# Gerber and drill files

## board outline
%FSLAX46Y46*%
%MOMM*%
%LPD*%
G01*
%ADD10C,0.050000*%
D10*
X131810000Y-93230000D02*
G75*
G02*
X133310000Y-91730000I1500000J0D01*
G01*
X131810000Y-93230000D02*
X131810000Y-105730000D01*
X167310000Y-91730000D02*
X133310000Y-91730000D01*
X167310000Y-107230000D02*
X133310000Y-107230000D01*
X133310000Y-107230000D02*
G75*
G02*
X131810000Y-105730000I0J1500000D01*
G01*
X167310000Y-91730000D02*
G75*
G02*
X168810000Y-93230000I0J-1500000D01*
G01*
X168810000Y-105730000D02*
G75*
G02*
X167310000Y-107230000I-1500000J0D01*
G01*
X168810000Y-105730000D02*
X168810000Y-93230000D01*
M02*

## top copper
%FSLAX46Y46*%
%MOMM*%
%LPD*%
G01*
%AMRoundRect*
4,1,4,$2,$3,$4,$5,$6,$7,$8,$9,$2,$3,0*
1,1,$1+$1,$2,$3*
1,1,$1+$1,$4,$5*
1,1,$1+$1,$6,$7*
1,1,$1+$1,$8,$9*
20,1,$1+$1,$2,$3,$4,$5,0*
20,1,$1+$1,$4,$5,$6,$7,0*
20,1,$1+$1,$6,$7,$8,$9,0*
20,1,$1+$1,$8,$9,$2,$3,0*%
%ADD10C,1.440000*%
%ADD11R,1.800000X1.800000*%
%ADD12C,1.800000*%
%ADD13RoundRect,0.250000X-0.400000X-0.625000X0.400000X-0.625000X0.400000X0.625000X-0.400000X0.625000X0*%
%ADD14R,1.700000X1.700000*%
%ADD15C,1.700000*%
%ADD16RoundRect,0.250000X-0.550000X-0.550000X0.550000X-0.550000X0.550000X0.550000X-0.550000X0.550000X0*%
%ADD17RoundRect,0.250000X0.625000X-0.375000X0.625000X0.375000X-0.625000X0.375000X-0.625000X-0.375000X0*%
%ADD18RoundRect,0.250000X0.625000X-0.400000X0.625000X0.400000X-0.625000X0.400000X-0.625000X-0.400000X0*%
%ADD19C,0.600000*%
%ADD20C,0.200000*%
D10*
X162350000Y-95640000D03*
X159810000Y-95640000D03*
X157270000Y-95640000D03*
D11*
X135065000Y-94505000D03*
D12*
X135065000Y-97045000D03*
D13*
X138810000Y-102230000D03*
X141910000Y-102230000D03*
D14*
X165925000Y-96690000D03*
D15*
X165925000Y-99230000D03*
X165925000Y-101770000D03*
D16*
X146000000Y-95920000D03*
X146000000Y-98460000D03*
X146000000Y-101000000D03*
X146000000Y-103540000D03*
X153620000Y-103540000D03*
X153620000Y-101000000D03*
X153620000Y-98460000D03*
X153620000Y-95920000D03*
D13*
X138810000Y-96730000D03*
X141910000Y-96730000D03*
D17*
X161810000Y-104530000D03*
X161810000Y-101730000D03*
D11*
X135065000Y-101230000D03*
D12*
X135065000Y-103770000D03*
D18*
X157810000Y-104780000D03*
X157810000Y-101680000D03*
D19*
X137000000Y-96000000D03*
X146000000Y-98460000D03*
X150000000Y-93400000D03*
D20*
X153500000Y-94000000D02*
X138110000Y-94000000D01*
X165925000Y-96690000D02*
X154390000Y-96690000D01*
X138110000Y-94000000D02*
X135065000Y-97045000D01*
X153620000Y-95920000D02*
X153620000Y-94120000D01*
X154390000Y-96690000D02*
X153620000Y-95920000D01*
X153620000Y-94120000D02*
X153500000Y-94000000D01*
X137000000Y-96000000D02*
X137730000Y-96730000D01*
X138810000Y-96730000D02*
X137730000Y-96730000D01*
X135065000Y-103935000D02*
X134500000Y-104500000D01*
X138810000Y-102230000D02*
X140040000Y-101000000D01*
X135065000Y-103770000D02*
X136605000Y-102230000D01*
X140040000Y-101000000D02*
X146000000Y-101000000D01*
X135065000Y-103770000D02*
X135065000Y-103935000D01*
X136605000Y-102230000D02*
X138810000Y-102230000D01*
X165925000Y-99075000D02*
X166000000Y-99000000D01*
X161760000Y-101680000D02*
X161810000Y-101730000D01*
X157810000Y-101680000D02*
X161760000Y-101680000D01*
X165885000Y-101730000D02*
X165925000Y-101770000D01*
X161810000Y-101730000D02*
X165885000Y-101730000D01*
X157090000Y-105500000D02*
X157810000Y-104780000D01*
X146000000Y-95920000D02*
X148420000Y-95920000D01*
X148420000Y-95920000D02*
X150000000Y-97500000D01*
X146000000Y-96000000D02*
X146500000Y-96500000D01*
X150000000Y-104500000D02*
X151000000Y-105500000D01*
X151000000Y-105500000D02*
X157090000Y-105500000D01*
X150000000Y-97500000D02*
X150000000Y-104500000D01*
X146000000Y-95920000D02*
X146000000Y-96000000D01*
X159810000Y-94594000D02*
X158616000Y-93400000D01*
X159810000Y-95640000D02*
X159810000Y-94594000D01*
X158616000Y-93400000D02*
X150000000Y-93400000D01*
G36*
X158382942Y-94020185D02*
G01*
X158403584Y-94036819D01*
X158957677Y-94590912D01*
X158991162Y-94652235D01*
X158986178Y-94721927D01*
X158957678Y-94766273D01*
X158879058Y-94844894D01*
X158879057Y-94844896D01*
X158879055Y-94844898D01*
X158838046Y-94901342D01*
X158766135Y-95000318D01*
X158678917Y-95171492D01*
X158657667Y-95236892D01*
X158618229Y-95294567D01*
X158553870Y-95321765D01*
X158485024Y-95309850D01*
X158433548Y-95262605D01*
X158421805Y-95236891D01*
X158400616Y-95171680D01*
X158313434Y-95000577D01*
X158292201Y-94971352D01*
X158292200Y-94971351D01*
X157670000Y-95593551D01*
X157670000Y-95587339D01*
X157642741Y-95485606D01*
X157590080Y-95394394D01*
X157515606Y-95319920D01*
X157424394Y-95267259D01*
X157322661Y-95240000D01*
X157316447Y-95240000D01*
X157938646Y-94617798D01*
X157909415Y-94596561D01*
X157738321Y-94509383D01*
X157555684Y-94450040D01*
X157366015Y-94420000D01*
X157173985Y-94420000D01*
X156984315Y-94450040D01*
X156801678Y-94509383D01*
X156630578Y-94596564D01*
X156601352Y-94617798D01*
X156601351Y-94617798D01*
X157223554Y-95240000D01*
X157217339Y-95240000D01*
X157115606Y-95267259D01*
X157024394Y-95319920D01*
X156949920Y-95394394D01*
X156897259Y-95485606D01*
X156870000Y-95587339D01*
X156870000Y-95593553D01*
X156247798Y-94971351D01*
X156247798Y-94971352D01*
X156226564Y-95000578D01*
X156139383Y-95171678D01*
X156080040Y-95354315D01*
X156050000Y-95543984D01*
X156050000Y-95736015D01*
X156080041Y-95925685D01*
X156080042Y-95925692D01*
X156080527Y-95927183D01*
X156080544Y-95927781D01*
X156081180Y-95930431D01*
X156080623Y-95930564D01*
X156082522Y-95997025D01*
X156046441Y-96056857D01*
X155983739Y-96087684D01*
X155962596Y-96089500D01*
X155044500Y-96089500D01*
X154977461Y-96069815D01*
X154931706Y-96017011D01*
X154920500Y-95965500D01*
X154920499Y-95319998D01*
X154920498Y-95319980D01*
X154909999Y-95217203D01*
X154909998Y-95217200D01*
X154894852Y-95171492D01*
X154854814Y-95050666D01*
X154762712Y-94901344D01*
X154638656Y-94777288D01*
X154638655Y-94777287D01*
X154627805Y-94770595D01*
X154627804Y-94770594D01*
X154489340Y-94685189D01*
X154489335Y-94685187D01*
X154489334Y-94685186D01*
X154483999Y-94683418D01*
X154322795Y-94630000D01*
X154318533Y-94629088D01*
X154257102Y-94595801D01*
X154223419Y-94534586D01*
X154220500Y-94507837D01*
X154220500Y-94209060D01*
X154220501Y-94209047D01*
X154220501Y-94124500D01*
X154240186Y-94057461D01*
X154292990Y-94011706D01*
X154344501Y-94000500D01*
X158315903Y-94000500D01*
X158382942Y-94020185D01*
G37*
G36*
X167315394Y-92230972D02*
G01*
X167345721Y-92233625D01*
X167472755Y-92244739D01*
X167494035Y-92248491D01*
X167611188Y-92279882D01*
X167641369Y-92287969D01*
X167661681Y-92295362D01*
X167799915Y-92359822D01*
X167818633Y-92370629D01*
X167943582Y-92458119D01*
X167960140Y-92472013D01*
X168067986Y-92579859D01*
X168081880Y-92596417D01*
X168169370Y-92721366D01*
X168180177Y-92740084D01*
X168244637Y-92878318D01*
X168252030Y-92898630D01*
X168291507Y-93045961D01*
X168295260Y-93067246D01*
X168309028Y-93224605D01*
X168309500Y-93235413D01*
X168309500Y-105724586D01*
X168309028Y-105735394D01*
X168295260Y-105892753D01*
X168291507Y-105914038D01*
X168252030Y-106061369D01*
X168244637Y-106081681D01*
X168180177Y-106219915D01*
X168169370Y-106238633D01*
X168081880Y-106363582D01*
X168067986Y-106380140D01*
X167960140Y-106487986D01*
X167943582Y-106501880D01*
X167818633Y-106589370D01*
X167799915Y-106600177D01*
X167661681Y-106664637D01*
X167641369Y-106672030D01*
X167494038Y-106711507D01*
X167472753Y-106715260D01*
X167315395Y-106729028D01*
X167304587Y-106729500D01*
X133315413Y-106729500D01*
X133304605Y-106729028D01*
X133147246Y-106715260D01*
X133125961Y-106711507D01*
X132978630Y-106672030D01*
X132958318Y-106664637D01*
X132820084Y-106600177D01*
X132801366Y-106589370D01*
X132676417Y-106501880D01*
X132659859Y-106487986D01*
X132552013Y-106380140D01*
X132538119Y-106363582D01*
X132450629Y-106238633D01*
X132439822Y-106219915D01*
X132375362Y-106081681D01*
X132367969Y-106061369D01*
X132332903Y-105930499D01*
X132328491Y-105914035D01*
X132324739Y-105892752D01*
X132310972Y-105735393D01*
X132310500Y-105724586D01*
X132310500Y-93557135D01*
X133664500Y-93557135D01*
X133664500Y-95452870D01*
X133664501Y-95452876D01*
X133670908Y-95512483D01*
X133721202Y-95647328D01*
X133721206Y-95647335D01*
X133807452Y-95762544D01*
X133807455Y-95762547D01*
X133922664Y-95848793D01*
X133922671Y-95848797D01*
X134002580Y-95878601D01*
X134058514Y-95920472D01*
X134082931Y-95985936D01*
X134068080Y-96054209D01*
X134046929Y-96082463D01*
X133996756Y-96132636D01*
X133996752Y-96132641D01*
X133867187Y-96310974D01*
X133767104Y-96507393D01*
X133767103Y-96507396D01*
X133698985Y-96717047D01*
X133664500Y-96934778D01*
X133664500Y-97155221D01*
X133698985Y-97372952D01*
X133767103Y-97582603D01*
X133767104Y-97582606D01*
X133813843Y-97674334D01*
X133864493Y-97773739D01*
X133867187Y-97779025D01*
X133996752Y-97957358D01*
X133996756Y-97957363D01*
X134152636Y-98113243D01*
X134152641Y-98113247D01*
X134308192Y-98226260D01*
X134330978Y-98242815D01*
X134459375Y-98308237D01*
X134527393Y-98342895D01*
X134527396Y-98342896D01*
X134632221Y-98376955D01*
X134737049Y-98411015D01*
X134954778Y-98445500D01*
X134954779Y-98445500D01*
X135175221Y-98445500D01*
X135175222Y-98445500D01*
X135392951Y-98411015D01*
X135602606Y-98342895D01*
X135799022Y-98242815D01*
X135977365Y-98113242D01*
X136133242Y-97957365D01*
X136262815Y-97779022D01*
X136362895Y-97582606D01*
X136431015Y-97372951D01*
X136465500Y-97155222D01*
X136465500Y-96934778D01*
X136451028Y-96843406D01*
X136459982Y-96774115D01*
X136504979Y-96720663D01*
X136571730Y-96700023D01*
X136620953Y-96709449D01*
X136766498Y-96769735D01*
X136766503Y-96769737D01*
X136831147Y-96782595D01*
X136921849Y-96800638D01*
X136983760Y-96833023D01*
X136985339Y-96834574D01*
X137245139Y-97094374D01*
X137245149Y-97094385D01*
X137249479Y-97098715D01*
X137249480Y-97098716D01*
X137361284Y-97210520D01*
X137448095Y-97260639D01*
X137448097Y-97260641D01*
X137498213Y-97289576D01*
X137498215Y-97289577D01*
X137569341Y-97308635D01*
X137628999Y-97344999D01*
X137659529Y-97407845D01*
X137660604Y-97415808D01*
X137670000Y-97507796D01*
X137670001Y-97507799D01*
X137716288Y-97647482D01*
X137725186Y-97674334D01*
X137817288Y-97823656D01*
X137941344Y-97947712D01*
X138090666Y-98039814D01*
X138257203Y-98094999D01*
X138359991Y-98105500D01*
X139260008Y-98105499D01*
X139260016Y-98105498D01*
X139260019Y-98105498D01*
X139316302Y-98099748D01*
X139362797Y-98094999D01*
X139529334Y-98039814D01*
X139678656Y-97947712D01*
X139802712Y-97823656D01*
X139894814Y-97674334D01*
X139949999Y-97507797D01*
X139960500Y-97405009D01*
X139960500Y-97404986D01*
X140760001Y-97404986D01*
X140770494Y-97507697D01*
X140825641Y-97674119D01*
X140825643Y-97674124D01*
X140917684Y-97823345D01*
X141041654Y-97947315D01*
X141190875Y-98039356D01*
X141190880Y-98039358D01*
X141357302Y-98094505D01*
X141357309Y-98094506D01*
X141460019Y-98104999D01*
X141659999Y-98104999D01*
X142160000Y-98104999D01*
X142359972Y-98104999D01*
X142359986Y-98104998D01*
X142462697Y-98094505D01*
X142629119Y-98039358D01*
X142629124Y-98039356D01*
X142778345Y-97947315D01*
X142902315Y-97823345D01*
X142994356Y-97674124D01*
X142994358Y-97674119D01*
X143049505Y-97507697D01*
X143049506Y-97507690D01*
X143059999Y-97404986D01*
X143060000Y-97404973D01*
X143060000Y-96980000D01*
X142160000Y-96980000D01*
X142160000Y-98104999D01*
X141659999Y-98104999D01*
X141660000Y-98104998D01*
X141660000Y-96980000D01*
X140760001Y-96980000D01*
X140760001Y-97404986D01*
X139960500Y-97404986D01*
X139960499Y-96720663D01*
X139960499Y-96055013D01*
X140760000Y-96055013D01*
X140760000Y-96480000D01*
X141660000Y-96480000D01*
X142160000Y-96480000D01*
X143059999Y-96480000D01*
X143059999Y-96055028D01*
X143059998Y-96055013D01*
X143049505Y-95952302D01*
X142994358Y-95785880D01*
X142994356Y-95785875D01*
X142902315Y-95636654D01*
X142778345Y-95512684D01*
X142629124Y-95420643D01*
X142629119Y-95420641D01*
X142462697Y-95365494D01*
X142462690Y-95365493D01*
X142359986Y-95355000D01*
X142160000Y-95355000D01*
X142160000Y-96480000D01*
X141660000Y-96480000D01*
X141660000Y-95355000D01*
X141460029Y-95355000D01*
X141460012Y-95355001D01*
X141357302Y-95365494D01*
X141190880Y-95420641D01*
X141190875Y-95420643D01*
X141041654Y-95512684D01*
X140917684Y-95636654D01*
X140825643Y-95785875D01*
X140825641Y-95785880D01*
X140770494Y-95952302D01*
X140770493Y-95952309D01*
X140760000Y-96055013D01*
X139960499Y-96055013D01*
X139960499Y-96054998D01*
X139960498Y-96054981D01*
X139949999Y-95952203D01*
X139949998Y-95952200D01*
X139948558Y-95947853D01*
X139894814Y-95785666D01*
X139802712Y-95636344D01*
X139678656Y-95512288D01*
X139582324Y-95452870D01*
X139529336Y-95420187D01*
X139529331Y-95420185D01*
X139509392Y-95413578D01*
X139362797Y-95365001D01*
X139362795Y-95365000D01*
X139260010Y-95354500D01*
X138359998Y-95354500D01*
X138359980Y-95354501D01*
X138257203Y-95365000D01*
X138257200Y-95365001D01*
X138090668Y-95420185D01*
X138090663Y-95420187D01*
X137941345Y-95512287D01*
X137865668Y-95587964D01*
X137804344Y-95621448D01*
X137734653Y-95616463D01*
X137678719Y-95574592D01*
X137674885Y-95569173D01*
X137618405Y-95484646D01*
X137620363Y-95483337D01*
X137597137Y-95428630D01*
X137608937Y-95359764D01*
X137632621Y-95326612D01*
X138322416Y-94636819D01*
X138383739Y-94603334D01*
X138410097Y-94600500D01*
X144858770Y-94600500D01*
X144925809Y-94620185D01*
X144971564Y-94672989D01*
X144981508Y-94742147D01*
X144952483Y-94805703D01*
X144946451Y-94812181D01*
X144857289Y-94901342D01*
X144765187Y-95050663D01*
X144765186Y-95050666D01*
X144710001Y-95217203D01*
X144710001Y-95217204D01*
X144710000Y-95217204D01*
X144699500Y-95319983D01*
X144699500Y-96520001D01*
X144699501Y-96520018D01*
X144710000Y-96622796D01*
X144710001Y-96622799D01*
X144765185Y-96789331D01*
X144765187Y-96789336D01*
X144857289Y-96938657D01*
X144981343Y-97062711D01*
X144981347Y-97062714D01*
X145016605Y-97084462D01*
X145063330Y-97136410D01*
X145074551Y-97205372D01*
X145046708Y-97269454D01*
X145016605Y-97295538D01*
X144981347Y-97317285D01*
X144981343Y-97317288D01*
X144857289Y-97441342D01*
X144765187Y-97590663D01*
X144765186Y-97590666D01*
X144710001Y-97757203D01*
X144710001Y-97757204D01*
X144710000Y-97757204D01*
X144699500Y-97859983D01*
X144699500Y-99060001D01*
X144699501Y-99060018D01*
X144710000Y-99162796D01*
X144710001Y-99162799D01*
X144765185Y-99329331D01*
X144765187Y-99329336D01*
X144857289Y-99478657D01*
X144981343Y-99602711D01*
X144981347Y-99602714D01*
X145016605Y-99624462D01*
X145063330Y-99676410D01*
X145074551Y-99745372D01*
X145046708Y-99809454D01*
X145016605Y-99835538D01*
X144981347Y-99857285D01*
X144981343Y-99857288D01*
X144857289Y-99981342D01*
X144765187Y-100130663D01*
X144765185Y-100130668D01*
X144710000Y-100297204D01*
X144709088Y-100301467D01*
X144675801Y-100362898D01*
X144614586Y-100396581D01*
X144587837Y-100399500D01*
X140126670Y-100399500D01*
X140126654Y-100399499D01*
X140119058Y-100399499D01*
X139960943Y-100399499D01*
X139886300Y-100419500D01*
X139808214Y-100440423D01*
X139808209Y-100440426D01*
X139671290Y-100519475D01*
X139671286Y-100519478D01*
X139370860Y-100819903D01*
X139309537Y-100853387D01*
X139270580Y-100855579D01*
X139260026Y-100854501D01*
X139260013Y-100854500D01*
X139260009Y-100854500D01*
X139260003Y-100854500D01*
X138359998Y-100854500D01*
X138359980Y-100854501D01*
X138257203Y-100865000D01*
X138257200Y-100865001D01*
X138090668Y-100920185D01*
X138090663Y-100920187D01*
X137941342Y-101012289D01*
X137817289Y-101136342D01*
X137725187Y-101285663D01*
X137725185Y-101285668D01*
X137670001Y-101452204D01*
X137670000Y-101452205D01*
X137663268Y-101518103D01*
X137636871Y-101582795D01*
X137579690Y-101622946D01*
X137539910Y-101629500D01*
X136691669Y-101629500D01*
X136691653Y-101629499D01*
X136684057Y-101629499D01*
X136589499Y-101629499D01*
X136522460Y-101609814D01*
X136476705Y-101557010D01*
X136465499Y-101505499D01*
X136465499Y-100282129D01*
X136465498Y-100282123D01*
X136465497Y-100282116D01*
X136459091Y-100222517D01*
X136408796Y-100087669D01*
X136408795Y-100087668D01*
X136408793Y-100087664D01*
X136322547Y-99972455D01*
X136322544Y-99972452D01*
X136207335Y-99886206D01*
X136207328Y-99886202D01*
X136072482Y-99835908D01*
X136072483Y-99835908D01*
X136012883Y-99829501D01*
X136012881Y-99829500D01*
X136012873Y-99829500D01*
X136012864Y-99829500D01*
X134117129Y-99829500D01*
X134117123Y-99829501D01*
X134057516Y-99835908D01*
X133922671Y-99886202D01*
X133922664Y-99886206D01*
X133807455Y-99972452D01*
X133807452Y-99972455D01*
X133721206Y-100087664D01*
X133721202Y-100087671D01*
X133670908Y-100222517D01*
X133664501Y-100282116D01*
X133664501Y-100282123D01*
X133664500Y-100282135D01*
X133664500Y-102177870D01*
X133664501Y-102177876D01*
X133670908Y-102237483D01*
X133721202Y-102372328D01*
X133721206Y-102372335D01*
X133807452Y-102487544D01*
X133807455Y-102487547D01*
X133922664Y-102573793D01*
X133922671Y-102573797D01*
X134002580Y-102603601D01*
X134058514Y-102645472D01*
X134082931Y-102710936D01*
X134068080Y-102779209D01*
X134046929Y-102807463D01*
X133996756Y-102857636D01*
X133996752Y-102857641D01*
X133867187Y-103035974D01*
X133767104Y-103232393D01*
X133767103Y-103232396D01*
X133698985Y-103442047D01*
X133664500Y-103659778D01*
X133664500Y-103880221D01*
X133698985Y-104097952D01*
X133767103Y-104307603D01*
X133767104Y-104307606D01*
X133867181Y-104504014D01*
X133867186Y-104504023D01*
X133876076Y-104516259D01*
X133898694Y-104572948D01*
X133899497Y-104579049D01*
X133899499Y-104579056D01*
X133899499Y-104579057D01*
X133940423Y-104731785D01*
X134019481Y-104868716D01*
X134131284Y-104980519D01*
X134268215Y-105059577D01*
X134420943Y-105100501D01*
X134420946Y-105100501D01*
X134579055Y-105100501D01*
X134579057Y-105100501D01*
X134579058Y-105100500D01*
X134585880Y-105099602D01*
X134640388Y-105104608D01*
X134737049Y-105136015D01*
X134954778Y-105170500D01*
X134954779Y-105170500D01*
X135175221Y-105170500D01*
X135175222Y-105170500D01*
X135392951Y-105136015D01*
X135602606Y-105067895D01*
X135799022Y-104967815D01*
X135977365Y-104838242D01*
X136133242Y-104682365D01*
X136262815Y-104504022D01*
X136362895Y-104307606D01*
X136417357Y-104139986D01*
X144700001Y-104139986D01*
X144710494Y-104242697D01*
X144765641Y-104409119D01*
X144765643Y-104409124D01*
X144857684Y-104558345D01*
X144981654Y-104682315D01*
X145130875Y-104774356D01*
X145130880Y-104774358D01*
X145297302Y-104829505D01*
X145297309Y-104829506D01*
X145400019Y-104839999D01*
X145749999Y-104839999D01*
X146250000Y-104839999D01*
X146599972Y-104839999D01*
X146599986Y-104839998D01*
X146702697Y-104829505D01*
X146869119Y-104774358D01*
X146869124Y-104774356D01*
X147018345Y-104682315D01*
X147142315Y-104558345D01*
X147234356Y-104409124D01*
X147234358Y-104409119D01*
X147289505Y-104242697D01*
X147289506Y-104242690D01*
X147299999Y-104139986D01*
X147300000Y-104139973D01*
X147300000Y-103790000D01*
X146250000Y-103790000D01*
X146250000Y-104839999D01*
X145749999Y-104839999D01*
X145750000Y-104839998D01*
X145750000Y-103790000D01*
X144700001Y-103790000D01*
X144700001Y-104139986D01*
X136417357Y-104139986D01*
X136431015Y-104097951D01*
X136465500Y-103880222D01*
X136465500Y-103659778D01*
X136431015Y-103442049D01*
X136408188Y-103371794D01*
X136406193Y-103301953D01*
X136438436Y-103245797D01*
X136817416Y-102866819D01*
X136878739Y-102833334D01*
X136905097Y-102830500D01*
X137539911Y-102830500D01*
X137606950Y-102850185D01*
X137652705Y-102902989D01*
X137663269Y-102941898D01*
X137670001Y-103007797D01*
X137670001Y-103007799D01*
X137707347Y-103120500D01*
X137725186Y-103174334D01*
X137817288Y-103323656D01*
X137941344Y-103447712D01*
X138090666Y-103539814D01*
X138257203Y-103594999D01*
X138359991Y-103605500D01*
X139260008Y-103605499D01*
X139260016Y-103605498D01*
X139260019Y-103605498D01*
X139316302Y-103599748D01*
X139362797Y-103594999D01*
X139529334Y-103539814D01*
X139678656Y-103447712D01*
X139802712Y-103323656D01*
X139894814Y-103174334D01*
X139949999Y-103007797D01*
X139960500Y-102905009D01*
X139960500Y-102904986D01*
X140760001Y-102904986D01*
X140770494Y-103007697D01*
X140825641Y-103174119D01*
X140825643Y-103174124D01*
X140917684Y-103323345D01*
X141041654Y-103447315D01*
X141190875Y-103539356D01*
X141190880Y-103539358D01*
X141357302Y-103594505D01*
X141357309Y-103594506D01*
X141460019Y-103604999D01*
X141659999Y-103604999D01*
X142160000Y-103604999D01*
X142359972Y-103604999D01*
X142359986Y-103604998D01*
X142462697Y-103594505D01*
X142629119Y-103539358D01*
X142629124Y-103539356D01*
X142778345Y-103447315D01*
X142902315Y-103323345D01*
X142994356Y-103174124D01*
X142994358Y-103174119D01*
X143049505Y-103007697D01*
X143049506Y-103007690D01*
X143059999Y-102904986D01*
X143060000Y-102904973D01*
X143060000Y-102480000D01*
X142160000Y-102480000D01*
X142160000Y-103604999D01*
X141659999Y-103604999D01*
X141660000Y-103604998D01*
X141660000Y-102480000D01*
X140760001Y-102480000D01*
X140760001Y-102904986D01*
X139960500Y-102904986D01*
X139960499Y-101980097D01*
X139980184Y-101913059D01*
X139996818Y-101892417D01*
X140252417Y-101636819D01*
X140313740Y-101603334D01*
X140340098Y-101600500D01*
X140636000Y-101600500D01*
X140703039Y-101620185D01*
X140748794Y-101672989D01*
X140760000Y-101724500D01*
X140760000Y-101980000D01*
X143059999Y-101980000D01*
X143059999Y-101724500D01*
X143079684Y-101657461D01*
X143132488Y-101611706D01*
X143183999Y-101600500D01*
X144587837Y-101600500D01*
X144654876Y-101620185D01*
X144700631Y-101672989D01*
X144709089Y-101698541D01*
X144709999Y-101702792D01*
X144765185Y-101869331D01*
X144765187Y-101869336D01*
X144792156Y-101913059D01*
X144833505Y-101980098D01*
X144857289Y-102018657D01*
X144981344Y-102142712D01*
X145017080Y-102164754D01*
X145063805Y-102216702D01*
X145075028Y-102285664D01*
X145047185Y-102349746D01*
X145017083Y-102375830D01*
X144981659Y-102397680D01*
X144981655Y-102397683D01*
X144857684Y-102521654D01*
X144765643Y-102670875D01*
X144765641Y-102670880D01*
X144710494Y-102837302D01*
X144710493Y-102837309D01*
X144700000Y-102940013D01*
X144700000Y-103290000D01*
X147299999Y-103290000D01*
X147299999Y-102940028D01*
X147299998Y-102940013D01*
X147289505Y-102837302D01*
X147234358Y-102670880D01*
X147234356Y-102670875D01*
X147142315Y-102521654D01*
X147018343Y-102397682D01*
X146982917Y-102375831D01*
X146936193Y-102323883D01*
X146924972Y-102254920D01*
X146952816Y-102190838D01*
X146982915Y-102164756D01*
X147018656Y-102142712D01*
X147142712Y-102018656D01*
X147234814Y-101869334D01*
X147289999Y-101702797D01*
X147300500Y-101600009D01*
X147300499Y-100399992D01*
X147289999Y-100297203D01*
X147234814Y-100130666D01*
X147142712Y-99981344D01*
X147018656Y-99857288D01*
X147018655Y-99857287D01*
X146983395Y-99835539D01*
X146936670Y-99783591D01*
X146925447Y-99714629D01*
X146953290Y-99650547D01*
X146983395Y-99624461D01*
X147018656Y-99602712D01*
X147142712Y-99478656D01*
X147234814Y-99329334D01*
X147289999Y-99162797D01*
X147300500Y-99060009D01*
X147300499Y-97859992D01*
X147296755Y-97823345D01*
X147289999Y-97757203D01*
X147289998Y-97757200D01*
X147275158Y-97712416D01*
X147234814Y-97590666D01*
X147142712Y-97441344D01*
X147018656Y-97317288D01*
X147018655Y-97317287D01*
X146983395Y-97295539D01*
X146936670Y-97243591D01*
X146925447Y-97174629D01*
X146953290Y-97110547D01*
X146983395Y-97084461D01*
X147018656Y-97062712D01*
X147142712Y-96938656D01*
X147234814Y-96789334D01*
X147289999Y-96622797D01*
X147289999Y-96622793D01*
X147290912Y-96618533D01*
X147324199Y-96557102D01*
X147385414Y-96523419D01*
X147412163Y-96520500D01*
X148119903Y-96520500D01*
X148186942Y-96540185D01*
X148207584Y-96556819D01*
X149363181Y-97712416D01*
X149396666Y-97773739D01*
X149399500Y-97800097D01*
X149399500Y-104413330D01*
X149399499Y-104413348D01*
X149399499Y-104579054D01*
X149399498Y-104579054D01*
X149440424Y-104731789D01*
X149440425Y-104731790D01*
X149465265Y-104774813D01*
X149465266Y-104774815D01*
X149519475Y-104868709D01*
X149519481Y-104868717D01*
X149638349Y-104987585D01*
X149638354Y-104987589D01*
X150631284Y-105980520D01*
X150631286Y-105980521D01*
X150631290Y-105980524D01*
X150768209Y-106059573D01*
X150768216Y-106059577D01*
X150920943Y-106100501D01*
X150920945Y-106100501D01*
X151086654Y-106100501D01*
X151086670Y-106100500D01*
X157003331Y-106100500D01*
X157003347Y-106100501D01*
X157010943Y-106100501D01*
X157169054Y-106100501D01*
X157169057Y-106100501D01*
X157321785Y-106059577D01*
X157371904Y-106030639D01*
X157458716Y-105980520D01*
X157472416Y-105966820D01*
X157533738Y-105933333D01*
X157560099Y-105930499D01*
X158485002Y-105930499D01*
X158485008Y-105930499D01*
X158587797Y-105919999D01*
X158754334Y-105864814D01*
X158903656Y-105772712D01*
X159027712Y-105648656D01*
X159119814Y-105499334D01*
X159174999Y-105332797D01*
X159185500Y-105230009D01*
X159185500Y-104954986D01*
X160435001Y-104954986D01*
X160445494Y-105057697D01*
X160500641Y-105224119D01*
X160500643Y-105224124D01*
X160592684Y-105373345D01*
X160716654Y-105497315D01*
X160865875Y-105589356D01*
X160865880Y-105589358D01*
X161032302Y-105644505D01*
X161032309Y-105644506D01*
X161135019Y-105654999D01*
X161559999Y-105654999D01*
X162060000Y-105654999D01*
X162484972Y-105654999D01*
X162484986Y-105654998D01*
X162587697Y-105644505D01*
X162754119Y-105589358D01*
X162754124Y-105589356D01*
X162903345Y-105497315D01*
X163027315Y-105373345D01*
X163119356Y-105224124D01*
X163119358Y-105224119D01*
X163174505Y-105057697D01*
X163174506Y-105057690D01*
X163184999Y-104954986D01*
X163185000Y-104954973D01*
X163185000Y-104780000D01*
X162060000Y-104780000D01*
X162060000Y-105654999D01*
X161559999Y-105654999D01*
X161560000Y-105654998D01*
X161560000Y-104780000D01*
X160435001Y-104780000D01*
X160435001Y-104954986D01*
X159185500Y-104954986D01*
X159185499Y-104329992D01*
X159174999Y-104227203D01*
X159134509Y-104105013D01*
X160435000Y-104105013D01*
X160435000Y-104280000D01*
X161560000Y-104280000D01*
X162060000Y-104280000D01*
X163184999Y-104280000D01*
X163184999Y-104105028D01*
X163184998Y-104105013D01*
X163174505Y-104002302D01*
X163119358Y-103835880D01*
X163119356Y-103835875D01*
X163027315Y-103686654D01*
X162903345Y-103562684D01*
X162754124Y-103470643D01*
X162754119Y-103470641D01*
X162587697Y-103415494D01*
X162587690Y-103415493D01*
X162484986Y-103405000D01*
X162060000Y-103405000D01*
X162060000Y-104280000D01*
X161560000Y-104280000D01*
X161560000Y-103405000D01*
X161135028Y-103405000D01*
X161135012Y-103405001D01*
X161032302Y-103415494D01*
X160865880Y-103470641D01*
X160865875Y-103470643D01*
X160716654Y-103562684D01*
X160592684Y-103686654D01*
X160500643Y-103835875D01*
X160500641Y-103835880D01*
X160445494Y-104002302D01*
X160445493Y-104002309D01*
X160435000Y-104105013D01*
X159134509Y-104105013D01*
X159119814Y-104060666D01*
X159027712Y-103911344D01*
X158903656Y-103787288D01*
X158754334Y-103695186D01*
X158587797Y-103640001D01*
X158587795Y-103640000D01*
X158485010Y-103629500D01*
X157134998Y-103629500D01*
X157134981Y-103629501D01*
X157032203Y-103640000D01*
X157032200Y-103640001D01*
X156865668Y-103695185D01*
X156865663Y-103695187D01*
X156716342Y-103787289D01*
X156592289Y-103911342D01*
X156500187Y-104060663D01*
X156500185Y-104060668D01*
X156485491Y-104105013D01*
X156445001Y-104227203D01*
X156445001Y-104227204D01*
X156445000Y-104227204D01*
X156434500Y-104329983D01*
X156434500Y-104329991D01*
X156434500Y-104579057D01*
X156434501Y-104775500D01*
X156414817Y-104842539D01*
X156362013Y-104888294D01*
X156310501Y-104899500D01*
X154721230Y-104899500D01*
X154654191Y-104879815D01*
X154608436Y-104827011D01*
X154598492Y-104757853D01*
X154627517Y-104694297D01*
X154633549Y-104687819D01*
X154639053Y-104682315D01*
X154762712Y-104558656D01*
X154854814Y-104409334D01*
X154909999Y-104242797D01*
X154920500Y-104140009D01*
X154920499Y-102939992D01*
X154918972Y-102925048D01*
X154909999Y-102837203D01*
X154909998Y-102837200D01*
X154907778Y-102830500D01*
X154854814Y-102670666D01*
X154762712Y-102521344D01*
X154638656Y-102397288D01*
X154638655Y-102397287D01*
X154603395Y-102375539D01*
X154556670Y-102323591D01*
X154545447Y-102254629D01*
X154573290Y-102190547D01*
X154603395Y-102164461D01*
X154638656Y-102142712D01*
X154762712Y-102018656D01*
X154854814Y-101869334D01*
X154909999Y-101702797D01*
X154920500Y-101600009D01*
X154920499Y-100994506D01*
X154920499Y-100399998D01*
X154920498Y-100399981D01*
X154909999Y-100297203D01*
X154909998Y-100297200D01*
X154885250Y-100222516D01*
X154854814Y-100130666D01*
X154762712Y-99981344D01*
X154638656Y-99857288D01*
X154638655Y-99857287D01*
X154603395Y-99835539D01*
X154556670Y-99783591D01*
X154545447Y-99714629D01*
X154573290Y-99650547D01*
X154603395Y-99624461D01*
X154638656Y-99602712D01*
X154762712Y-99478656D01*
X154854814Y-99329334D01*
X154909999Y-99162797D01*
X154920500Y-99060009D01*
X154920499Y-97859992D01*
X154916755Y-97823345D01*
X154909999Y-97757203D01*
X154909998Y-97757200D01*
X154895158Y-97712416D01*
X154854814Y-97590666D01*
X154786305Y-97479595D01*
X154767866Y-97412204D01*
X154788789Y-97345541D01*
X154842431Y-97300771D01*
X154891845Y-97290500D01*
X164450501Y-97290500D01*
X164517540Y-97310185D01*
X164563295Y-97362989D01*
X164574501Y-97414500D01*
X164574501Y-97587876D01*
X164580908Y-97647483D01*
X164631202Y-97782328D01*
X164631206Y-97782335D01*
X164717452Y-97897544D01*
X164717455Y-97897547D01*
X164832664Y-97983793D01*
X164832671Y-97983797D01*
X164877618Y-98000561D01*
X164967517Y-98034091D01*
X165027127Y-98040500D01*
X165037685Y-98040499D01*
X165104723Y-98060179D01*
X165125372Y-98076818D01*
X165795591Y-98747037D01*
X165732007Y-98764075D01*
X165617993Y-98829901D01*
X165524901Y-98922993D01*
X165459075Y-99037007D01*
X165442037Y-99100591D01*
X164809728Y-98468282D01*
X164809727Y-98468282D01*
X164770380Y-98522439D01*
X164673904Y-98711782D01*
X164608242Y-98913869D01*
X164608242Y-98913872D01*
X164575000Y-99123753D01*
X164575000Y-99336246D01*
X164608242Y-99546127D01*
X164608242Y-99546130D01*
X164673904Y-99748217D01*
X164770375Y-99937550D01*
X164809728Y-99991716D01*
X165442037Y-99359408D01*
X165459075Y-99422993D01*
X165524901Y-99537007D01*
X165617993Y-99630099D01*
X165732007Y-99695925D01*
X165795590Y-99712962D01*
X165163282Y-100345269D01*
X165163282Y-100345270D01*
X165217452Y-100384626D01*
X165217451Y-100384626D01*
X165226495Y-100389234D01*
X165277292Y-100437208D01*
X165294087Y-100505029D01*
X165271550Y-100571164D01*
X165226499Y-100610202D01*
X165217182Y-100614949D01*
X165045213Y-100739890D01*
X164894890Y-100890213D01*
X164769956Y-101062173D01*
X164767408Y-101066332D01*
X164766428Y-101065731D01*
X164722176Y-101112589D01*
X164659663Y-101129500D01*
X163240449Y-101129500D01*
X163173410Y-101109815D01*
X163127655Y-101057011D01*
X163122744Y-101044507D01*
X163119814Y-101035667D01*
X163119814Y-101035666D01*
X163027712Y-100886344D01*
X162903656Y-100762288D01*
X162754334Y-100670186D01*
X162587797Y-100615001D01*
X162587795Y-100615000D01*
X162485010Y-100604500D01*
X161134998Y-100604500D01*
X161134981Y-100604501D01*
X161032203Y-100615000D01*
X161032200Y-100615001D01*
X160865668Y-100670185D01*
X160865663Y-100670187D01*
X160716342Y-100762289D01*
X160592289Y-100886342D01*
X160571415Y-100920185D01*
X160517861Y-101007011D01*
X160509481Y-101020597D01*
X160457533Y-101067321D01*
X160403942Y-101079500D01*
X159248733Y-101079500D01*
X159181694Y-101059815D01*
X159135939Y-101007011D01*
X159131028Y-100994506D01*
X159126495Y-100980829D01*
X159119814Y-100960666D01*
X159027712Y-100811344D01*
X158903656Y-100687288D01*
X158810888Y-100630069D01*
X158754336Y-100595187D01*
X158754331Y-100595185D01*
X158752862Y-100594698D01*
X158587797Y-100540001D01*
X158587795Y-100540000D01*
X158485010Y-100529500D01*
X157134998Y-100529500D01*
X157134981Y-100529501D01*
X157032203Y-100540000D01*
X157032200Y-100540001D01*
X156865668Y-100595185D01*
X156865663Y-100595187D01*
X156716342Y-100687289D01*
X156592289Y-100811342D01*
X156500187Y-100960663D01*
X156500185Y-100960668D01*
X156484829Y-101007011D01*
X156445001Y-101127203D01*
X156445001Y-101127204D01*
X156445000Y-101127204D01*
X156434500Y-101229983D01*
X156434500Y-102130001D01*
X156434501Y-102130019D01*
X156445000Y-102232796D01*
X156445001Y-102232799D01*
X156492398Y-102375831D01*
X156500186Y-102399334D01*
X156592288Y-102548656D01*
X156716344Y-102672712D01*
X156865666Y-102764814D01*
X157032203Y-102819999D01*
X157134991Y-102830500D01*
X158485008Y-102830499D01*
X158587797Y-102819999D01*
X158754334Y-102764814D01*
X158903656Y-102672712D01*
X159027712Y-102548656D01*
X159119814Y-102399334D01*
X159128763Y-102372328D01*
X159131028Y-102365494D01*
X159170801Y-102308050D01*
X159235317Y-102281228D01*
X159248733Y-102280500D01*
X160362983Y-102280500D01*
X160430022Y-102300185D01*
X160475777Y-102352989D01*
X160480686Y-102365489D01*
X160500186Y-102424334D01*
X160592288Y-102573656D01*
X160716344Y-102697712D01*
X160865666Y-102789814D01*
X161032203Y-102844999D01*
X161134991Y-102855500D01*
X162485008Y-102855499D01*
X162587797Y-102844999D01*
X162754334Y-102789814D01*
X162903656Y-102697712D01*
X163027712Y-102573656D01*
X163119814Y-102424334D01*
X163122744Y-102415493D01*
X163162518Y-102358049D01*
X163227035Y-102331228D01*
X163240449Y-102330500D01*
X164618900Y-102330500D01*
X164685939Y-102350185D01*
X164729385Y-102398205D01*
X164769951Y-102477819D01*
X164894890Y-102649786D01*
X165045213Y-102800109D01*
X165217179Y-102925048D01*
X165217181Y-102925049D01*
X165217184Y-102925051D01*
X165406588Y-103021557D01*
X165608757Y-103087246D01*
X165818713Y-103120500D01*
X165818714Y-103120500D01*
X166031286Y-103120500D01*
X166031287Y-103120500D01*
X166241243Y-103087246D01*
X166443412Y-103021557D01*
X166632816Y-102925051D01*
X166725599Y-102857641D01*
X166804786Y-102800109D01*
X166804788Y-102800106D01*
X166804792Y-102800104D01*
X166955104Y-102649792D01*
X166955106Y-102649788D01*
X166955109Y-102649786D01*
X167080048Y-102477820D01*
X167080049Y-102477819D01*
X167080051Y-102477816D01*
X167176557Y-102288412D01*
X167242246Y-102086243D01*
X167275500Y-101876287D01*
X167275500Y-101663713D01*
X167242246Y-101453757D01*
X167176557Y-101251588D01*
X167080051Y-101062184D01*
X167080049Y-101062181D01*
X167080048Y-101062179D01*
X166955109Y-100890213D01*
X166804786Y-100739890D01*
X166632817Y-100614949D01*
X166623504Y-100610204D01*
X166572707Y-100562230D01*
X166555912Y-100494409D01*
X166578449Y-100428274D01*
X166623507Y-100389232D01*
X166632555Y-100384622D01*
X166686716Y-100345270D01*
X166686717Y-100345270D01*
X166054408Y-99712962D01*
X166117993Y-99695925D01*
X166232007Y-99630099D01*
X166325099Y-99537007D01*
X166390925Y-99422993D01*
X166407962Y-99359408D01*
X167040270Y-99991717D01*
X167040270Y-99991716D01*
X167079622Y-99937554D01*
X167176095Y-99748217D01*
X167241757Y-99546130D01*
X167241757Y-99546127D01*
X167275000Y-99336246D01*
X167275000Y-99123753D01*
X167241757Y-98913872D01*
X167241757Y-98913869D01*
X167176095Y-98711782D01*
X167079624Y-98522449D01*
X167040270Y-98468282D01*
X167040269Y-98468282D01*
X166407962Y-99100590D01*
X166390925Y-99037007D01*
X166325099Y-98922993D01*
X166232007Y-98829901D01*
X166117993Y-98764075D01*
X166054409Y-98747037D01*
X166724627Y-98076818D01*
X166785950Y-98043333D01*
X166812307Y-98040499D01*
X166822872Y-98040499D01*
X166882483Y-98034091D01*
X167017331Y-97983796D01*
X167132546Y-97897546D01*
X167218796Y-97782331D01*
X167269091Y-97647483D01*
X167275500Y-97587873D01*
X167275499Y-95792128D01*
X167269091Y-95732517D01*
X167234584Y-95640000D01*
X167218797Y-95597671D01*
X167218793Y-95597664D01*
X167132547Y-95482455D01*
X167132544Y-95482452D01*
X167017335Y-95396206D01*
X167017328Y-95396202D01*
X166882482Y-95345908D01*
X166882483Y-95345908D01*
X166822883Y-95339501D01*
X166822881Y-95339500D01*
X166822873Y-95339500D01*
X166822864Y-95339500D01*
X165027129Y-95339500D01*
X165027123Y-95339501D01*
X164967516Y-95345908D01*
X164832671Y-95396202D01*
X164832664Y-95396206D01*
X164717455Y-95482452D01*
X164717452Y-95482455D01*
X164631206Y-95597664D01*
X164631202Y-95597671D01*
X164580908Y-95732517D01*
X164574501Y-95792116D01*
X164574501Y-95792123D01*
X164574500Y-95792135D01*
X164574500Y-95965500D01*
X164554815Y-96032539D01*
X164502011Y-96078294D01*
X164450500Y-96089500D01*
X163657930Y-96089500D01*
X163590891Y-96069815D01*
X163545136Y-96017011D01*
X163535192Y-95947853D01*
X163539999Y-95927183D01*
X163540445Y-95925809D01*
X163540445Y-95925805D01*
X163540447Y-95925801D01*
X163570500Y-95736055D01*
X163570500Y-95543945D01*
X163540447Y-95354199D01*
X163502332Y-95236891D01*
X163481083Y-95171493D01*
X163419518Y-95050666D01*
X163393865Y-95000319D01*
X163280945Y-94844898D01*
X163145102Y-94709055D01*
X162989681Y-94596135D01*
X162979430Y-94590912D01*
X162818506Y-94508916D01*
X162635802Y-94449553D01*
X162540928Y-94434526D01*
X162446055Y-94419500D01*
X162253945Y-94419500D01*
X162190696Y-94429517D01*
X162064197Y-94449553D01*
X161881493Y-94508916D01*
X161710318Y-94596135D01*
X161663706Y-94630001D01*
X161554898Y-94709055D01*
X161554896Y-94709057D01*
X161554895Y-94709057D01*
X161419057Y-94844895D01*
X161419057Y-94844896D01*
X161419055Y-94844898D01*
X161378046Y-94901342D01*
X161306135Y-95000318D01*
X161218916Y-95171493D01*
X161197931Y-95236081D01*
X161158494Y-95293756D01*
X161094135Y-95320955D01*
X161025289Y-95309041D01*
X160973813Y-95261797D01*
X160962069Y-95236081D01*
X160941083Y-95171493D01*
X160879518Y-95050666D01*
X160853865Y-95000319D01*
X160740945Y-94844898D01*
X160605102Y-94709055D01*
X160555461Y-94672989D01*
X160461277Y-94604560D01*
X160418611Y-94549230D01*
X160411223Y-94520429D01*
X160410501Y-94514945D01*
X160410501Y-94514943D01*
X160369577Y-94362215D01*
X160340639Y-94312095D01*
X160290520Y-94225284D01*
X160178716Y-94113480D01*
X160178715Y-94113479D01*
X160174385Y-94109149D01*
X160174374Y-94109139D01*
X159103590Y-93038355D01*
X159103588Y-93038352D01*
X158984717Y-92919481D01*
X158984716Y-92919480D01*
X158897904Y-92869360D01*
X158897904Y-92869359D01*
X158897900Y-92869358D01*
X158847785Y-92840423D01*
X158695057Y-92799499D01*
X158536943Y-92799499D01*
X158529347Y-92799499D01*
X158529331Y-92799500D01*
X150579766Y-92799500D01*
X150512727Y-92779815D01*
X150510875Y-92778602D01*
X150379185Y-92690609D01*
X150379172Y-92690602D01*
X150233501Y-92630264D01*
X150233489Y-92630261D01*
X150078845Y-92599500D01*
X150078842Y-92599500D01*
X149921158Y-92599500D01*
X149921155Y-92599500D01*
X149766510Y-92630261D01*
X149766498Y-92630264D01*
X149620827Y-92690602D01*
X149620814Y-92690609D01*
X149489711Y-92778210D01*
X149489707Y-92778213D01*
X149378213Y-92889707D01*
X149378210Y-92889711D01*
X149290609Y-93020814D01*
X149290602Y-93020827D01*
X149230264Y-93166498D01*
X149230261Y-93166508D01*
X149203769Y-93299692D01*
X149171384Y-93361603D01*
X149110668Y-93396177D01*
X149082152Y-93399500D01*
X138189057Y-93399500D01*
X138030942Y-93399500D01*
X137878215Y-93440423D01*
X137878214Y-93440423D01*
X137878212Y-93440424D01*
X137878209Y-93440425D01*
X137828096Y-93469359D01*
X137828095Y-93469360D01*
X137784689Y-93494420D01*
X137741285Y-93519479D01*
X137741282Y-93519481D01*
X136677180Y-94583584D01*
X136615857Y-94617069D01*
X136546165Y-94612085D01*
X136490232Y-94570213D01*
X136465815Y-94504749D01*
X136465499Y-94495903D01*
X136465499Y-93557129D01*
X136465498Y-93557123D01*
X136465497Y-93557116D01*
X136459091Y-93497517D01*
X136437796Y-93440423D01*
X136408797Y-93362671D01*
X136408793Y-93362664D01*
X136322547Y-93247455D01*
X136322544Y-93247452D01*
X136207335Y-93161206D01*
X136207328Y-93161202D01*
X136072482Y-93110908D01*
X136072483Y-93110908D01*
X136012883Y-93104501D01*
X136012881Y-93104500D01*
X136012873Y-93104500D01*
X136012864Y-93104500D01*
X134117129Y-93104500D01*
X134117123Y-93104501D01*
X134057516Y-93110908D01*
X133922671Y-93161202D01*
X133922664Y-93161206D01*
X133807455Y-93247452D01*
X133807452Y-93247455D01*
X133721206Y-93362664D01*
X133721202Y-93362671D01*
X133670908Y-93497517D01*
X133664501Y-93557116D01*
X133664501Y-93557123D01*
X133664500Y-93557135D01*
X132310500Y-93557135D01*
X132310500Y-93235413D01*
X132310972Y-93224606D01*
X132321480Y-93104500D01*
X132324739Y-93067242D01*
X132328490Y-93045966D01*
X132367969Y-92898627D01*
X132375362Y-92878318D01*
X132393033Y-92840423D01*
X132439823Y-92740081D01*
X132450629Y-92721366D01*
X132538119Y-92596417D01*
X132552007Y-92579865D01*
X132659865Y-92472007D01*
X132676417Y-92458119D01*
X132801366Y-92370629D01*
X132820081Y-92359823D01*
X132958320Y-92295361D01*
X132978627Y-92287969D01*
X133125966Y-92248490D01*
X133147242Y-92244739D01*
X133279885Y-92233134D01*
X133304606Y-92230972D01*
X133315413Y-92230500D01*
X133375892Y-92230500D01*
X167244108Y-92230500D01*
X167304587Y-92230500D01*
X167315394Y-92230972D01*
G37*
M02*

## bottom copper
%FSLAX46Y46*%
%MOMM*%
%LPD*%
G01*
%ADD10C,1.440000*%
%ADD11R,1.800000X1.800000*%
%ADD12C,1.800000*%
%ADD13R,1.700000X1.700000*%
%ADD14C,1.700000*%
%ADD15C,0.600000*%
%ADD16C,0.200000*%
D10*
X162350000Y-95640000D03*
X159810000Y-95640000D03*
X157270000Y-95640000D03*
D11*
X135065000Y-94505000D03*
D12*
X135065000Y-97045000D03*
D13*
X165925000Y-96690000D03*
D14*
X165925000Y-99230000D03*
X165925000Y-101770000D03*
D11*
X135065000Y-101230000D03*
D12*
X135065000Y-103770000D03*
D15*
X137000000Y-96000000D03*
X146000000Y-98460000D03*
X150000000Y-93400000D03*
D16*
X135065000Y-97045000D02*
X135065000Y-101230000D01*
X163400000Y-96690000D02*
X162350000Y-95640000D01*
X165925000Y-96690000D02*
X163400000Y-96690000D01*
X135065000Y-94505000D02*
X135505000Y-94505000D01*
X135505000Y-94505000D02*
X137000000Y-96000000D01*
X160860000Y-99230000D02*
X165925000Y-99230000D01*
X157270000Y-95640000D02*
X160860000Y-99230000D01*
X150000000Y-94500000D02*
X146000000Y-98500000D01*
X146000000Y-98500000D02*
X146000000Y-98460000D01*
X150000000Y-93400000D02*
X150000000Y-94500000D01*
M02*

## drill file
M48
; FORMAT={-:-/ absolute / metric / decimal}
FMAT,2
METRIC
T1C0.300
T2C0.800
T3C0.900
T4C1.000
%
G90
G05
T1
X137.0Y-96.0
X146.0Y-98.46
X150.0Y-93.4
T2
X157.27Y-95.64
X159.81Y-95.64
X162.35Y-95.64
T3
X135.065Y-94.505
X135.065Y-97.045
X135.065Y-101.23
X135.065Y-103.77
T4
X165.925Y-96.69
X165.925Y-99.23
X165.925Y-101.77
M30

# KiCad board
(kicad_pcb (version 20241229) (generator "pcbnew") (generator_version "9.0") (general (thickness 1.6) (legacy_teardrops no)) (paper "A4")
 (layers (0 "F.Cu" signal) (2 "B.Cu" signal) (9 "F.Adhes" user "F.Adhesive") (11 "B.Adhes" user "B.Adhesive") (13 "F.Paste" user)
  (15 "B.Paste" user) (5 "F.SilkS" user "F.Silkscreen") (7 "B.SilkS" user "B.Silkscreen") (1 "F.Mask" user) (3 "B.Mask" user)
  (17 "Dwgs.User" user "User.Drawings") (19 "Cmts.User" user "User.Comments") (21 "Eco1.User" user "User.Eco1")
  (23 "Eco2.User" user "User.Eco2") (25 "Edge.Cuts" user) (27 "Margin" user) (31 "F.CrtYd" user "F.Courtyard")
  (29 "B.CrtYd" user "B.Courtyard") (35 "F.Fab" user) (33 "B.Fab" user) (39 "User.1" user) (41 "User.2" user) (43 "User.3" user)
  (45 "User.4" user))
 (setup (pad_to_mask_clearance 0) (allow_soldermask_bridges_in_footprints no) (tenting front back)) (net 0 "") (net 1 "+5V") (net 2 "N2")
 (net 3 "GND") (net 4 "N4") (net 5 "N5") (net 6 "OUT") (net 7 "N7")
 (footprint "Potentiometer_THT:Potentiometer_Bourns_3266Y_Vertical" (layer "F.Cu") (at 162.35 95.64)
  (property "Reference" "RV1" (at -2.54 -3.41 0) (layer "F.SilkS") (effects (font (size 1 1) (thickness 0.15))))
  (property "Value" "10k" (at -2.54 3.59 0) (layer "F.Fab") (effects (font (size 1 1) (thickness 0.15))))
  (pad "1" thru_hole circle (at 0 0) (size 1.44 1.44) (drill 0.8) (layers "*.Cu" "*.Mask") (remove_unused_layers no) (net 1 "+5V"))
  (pad "2" thru_hole circle (at -2.54 0) (size 1.44 1.44) (drill 0.8) (layers "*.Cu" "*.Mask") (remove_unused_layers no) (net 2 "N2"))
  (pad "3" thru_hole circle (at -5.08 0) (size 1.44 1.44) (drill 0.8) (layers "*.Cu" "*.Mask") (remove_unused_layers no) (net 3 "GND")))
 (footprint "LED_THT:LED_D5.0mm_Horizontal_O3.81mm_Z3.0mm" (layer "F.Cu") (at 135.065 94.505 -90)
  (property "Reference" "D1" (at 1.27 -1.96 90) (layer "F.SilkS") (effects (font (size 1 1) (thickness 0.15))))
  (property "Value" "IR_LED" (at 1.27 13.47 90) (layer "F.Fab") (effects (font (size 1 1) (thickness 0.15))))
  (pad "1" thru_hole rect (at 0 0 270) (size 1.8 1.8) (drill 0.9) (layers "*.Cu" "*.Mask") (remove_unused_layers no) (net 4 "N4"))
  (pad "2" thru_hole circle (at 2.54 0 270) (size 1.8 1.8) (drill 0.9) (layers "*.Cu" "*.Mask") (remove_unused_layers no) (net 1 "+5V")))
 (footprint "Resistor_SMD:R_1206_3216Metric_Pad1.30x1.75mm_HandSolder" (layer "F.Cu") (at 140.36 102.23)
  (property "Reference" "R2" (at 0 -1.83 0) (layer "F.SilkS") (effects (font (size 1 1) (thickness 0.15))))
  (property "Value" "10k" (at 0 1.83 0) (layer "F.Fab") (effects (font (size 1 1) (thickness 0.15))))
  (pad "1" smd roundrect (at -1.55 0) (size 1.3 1.75) (layers "F.Cu" "F.Mask" "F.Paste") (roundrect_rratio 0.192308) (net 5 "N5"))
  (pad "2" smd roundrect (at 1.55 0) (size 1.3 1.75) (layers "F.Cu" "F.Mask" "F.Paste") (roundrect_rratio 0.192308) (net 3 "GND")))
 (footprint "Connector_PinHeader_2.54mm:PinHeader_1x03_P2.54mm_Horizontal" (layer "F.Cu") (at 165.925 96.69)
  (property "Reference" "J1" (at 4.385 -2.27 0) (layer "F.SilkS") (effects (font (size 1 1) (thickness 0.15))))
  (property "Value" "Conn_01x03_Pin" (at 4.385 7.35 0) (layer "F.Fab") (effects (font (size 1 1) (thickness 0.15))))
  (pad "1" thru_hole rect (at 0 0) (size 1.7 1.7) (drill 1) (layers "*.Cu" "*.Mask") (remove_unused_layers no) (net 1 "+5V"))
  (pad "2" thru_hole circle (at 0 2.54) (size 1.7 1.7) (drill 1) (layers "*.Cu" "*.Mask") (remove_unused_layers no) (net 3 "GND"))
  (pad "3" thru_hole circle (at 0 5.08) (size 1.7 1.7) (drill 1) (layers "*.Cu" "*.Mask") (remove_unused_layers no) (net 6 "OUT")))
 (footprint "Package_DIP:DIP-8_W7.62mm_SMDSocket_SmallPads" (layer "F.Cu") (at 149.81 99.73)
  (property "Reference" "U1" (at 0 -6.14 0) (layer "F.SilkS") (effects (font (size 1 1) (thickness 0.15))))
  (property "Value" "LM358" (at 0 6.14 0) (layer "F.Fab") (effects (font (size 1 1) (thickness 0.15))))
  (pad "1" smd roundrect (at -3.81 -3.81) (size 1.6 1.6) (layers "F.Cu" "F.Mask" "F.Paste") (roundrect_rratio 0.15625) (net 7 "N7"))
  (pad "2" smd roundrect (at -3.81 -1.27) (size 1.6 1.6) (layers "F.Cu" "F.Mask" "F.Paste") (roundrect_rratio 0.15625) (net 2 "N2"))
  (pad "3" smd roundrect (at -3.81 1.27) (size 1.6 1.6) (layers "F.Cu" "F.Mask" "F.Paste") (roundrect_rratio 0.15625) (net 5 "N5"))
  (pad "4" smd roundrect (at -3.81 3.81) (size 1.6 1.6) (layers "F.Cu" "F.Mask" "F.Paste") (roundrect_rratio 0.15625) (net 3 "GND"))
  (pad "5" smd roundrect (at 3.81 3.81) (size 1.6 1.6) (layers "F.Cu" "F.Mask" "F.Paste") (roundrect_rratio 0.15625))
  (pad "6" smd roundrect (at 3.81 1.27) (size 1.6 1.6) (layers "F.Cu" "F.Mask" "F.Paste") (roundrect_rratio 0.15625))
  (pad "7" smd roundrect (at 3.81 -1.27) (size 1.6 1.6) (layers "F.Cu" "F.Mask" "F.Paste") (roundrect_rratio 0.15625))
  (pad "8" smd roundrect (at 3.81 -3.81) (size 1.6 1.6) (layers "F.Cu" "F.Mask" "F.Paste") (roundrect_rratio 0.15625) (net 1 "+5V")))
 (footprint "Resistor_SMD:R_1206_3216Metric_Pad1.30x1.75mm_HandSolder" (layer "F.Cu") (at 140.36 96.73)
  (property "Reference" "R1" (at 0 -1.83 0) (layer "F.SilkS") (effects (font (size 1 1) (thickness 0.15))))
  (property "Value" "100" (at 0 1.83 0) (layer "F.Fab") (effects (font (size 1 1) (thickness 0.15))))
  (pad "1" smd roundrect (at -1.55 0) (size 1.3 1.75) (layers "F.Cu" "F.Mask" "F.Paste") (roundrect_rratio 0.192308) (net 4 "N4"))
  (pad "2" smd roundrect (at 1.55 0) (size 1.3 1.75) (layers "F.Cu" "F.Mask" "F.Paste") (roundrect_rratio 0.192308) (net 3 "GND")))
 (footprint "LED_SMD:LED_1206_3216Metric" (layer "F.Cu") (at 161.81 103.13 90)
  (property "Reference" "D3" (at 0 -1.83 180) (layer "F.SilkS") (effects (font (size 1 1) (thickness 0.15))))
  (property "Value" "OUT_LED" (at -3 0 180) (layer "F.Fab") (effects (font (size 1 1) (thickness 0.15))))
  (pad "1" smd roundrect (at -1.4 0 90) (size 1.25 1.75) (layers "F.Cu" "F.Mask" "F.Paste") (roundrect_rratio 0.2) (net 3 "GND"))
  (pad "2" smd roundrect (at 1.4 0 90) (size 1.25 1.75) (layers "F.Cu" "F.Mask" "F.Paste") (roundrect_rratio 0.2) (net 6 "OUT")))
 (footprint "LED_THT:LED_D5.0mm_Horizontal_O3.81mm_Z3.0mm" (layer "F.Cu") (at 135.065 101.23 -90)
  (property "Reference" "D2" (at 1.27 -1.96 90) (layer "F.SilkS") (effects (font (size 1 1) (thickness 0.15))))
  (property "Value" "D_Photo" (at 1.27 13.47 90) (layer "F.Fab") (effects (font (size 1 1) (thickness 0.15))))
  (pad "1" thru_hole rect (at 0 0 270) (size 1.8 1.8) (drill 0.9) (layers "*.Cu" "*.Mask") (remove_unused_layers no) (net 1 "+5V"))
  (pad "2" thru_hole circle (at 2.54 0 270) (size 1.8 1.8) (drill 0.9) (layers "*.Cu" "*.Mask") (remove_unused_layers no) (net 5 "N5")))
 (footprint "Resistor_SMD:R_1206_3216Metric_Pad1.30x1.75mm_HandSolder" (layer "F.Cu") (at 157.81 103.23 90)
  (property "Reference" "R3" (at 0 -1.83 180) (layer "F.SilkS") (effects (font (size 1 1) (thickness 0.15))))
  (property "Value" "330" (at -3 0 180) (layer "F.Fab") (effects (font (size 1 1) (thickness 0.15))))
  (pad "1" smd roundrect (at -1.55 0 90) (size 1.3 1.75) (layers "F.Cu" "F.Mask" "F.Paste") (roundrect_rratio 0.192308) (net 7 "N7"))
  (pad "2" smd roundrect (at 1.55 0 90) (size 1.3 1.75) (layers "F.Cu" "F.Mask" "F.Paste") (roundrect_rratio 0.192308) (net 6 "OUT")))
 (gr_arc (start 131.81 93.23) (mid 132.24934 92.16934) (end 133.31 91.73) (stroke (width 0.05) (type default)) (layer "Edge.Cuts"))
 (gr_line (start 131.81 93.23) (end 131.81 105.73) (stroke (width 0.05) (type default)) (layer "Edge.Cuts"))
 (gr_line (start 167.31 91.73) (end 133.31 91.73) (stroke (width 0.05) (type default)) (layer "Edge.Cuts"))
 (gr_line (start 167.31 107.23) (end 133.31 107.23) (stroke (width 0.05) (type default)) (layer "Edge.Cuts"))
 (gr_arc (start 133.31 107.23) (mid 132.24934 106.79066) (end 131.81 105.73) (stroke (width 0.05) (type default)) (layer "Edge.Cuts"))
 (gr_arc (start 167.31 91.73) (mid 168.37066 92.16934) (end 168.81 93.23) (stroke (width 0.05) (type default)) (layer "Edge.Cuts"))
 (gr_arc (start 168.81 105.73) (mid 168.37066 106.79066) (end 167.31 107.23) (stroke (width 0.05) (type default)) (layer "Edge.Cuts"))
 (gr_line (start 168.81 105.73) (end 168.81 93.23) (stroke (width 0.05) (type default)) (layer "Edge.Cuts"))
 (segment (start 153.5 94) (end 138.11 94) (width 0.2) (layer "F.Cu") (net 1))
 (segment (start 165.925 96.69) (end 154.39 96.69) (width 0.2) (layer "F.Cu") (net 1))
 (segment (start 138.11 94) (end 135.065 97.045) (width 0.2) (layer "F.Cu") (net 1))
 (segment (start 153.62 95.92) (end 153.62 94.12) (width 0.2) (layer "F.Cu") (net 1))
 (segment (start 154.39 96.69) (end 153.62 95.92) (width 0.2) (layer "F.Cu") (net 1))
 (segment (start 153.62 94.12) (end 153.5 94) (width 0.2) (layer "F.Cu") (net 1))
 (segment (start 135.065 97.045) (end 135.065 101.23) (width 0.2) (layer "B.Cu") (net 1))
 (segment (start 163.4 96.69) (end 162.35 95.64) (width 0.2) (layer "B.Cu") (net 1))
 (segment (start 165.925 96.69) (end 163.4 96.69) (width 0.2) (layer "B.Cu") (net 1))
 (segment (start 137 96) (end 137.73 96.73) (width 0.2) (layer "F.Cu") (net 4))
 (segment (start 138.81 96.73) (end 137.73 96.73) (width 0.2) (layer "F.Cu") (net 4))
 (via (at 137 96) (size 0.6) (drill 0.3) (layers "F.Cu" "B.Cu") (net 4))
 (segment (start 135.065 94.505) (end 135.505 94.505) (width 0.2) (layer "B.Cu") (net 4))
 (segment (start 135.505 94.505) (end 137 96) (width 0.2) (layer "B.Cu") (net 4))
 (segment (start 135.065 103.935) (end 134.5 104.5) (width 0.2) (layer "F.Cu") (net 5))
 (segment (start 138.81 102.23) (end 140.04 101) (width 0.2) (layer "F.Cu") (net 5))
 (segment (start 135.065 103.77) (end 136.605 102.23) (width 0.2) (layer "F.Cu") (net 5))
 (segment (start 140.04 101) (end 146 101) (width 0.2) (layer "F.Cu") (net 5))
 (segment (start 135.065 103.77) (end 135.065 103.935) (width 0.2) (layer "F.Cu") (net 5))
 (segment (start 136.605 102.23) (end 138.81 102.23) (width 0.2) (layer "F.Cu") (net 5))
 (segment (start 165.925 99.075) (end 166 99) (width 0.2) (layer "F.Cu") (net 3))
 (segment (start 160.86 99.23) (end 165.925 99.23) (width 0.2) (layer "B.Cu") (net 3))
 (segment (start 157.27 95.64) (end 160.86 99.23) (width 0.2) (layer "B.Cu") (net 3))
 (segment (start 161.76 101.68) (end 161.81 101.73) (width 0.2) (layer "F.Cu") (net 6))
 (segment (start 157.81 101.68) (end 161.76 101.68) (width 0.2) (layer "F.Cu") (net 6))
 (segment (start 165.885 101.73) (end 165.925 101.77) (width 0.2) (layer "F.Cu") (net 6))
 (segment (start 161.81 101.73) (end 165.885 101.73) (width 0.2) (layer "F.Cu") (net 6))
 (segment (start 157.09 105.5) (end 157.81 104.78) (width 0.2) (layer "F.Cu") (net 7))
 (segment (start 146 95.92) (end 148.42 95.92) (width 0.2) (layer "F.Cu") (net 7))
 (segment (start 148.42 95.92) (end 150 97.5) (width 0.2) (layer "F.Cu") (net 7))
 (segment (start 146 96) (end 146.5 96.5) (width 0.2) (layer "F.Cu") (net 7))
 (segment (start 150 104.5) (end 151 105.5) (width 0.2) (layer "F.Cu") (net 7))
 (segment (start 151 105.5) (end 157.09 105.5) (width 0.2) (layer "F.Cu") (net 7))
 (segment (start 150 97.5) (end 150 104.5) (width 0.2) (layer "F.Cu") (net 7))
 (segment (start 146 95.92) (end 146 96) (width 0.2) (layer "F.Cu") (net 7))
 (segment (start 159.81 94.594) (end 158.616 93.4) (width 0.2) (layer "F.Cu") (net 2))
 (segment (start 159.81 95.64) (end 159.81 94.594) (width 0.2) (layer "F.Cu") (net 2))
 (segment (start 158.616 93.4) (end 150 93.4) (width 0.2) (layer "F.Cu") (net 2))
 (via (at 146 98.46) (size 0.6) (drill 0.3) (layers "F.Cu" "B.Cu") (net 2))
 (via (at 150 93.4) (size 0.6) (drill 0.3) (layers "F.Cu" "B.Cu") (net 2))
 (segment (start 150 94.5) (end 146 98.5) (width 0.2) (layer "B.Cu") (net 2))
 (segment (start 146 98.5) (end 146 98.46) (width 0.2) (layer "B.Cu") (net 2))
 (segment (start 150 93.4) (end 150 94.5) (width 0.2) (layer "B.Cu") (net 2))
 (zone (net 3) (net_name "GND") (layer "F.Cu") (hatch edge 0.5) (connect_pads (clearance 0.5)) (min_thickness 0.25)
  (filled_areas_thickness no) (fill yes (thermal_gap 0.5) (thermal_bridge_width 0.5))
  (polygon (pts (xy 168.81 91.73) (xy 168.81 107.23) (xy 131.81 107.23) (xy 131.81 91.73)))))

